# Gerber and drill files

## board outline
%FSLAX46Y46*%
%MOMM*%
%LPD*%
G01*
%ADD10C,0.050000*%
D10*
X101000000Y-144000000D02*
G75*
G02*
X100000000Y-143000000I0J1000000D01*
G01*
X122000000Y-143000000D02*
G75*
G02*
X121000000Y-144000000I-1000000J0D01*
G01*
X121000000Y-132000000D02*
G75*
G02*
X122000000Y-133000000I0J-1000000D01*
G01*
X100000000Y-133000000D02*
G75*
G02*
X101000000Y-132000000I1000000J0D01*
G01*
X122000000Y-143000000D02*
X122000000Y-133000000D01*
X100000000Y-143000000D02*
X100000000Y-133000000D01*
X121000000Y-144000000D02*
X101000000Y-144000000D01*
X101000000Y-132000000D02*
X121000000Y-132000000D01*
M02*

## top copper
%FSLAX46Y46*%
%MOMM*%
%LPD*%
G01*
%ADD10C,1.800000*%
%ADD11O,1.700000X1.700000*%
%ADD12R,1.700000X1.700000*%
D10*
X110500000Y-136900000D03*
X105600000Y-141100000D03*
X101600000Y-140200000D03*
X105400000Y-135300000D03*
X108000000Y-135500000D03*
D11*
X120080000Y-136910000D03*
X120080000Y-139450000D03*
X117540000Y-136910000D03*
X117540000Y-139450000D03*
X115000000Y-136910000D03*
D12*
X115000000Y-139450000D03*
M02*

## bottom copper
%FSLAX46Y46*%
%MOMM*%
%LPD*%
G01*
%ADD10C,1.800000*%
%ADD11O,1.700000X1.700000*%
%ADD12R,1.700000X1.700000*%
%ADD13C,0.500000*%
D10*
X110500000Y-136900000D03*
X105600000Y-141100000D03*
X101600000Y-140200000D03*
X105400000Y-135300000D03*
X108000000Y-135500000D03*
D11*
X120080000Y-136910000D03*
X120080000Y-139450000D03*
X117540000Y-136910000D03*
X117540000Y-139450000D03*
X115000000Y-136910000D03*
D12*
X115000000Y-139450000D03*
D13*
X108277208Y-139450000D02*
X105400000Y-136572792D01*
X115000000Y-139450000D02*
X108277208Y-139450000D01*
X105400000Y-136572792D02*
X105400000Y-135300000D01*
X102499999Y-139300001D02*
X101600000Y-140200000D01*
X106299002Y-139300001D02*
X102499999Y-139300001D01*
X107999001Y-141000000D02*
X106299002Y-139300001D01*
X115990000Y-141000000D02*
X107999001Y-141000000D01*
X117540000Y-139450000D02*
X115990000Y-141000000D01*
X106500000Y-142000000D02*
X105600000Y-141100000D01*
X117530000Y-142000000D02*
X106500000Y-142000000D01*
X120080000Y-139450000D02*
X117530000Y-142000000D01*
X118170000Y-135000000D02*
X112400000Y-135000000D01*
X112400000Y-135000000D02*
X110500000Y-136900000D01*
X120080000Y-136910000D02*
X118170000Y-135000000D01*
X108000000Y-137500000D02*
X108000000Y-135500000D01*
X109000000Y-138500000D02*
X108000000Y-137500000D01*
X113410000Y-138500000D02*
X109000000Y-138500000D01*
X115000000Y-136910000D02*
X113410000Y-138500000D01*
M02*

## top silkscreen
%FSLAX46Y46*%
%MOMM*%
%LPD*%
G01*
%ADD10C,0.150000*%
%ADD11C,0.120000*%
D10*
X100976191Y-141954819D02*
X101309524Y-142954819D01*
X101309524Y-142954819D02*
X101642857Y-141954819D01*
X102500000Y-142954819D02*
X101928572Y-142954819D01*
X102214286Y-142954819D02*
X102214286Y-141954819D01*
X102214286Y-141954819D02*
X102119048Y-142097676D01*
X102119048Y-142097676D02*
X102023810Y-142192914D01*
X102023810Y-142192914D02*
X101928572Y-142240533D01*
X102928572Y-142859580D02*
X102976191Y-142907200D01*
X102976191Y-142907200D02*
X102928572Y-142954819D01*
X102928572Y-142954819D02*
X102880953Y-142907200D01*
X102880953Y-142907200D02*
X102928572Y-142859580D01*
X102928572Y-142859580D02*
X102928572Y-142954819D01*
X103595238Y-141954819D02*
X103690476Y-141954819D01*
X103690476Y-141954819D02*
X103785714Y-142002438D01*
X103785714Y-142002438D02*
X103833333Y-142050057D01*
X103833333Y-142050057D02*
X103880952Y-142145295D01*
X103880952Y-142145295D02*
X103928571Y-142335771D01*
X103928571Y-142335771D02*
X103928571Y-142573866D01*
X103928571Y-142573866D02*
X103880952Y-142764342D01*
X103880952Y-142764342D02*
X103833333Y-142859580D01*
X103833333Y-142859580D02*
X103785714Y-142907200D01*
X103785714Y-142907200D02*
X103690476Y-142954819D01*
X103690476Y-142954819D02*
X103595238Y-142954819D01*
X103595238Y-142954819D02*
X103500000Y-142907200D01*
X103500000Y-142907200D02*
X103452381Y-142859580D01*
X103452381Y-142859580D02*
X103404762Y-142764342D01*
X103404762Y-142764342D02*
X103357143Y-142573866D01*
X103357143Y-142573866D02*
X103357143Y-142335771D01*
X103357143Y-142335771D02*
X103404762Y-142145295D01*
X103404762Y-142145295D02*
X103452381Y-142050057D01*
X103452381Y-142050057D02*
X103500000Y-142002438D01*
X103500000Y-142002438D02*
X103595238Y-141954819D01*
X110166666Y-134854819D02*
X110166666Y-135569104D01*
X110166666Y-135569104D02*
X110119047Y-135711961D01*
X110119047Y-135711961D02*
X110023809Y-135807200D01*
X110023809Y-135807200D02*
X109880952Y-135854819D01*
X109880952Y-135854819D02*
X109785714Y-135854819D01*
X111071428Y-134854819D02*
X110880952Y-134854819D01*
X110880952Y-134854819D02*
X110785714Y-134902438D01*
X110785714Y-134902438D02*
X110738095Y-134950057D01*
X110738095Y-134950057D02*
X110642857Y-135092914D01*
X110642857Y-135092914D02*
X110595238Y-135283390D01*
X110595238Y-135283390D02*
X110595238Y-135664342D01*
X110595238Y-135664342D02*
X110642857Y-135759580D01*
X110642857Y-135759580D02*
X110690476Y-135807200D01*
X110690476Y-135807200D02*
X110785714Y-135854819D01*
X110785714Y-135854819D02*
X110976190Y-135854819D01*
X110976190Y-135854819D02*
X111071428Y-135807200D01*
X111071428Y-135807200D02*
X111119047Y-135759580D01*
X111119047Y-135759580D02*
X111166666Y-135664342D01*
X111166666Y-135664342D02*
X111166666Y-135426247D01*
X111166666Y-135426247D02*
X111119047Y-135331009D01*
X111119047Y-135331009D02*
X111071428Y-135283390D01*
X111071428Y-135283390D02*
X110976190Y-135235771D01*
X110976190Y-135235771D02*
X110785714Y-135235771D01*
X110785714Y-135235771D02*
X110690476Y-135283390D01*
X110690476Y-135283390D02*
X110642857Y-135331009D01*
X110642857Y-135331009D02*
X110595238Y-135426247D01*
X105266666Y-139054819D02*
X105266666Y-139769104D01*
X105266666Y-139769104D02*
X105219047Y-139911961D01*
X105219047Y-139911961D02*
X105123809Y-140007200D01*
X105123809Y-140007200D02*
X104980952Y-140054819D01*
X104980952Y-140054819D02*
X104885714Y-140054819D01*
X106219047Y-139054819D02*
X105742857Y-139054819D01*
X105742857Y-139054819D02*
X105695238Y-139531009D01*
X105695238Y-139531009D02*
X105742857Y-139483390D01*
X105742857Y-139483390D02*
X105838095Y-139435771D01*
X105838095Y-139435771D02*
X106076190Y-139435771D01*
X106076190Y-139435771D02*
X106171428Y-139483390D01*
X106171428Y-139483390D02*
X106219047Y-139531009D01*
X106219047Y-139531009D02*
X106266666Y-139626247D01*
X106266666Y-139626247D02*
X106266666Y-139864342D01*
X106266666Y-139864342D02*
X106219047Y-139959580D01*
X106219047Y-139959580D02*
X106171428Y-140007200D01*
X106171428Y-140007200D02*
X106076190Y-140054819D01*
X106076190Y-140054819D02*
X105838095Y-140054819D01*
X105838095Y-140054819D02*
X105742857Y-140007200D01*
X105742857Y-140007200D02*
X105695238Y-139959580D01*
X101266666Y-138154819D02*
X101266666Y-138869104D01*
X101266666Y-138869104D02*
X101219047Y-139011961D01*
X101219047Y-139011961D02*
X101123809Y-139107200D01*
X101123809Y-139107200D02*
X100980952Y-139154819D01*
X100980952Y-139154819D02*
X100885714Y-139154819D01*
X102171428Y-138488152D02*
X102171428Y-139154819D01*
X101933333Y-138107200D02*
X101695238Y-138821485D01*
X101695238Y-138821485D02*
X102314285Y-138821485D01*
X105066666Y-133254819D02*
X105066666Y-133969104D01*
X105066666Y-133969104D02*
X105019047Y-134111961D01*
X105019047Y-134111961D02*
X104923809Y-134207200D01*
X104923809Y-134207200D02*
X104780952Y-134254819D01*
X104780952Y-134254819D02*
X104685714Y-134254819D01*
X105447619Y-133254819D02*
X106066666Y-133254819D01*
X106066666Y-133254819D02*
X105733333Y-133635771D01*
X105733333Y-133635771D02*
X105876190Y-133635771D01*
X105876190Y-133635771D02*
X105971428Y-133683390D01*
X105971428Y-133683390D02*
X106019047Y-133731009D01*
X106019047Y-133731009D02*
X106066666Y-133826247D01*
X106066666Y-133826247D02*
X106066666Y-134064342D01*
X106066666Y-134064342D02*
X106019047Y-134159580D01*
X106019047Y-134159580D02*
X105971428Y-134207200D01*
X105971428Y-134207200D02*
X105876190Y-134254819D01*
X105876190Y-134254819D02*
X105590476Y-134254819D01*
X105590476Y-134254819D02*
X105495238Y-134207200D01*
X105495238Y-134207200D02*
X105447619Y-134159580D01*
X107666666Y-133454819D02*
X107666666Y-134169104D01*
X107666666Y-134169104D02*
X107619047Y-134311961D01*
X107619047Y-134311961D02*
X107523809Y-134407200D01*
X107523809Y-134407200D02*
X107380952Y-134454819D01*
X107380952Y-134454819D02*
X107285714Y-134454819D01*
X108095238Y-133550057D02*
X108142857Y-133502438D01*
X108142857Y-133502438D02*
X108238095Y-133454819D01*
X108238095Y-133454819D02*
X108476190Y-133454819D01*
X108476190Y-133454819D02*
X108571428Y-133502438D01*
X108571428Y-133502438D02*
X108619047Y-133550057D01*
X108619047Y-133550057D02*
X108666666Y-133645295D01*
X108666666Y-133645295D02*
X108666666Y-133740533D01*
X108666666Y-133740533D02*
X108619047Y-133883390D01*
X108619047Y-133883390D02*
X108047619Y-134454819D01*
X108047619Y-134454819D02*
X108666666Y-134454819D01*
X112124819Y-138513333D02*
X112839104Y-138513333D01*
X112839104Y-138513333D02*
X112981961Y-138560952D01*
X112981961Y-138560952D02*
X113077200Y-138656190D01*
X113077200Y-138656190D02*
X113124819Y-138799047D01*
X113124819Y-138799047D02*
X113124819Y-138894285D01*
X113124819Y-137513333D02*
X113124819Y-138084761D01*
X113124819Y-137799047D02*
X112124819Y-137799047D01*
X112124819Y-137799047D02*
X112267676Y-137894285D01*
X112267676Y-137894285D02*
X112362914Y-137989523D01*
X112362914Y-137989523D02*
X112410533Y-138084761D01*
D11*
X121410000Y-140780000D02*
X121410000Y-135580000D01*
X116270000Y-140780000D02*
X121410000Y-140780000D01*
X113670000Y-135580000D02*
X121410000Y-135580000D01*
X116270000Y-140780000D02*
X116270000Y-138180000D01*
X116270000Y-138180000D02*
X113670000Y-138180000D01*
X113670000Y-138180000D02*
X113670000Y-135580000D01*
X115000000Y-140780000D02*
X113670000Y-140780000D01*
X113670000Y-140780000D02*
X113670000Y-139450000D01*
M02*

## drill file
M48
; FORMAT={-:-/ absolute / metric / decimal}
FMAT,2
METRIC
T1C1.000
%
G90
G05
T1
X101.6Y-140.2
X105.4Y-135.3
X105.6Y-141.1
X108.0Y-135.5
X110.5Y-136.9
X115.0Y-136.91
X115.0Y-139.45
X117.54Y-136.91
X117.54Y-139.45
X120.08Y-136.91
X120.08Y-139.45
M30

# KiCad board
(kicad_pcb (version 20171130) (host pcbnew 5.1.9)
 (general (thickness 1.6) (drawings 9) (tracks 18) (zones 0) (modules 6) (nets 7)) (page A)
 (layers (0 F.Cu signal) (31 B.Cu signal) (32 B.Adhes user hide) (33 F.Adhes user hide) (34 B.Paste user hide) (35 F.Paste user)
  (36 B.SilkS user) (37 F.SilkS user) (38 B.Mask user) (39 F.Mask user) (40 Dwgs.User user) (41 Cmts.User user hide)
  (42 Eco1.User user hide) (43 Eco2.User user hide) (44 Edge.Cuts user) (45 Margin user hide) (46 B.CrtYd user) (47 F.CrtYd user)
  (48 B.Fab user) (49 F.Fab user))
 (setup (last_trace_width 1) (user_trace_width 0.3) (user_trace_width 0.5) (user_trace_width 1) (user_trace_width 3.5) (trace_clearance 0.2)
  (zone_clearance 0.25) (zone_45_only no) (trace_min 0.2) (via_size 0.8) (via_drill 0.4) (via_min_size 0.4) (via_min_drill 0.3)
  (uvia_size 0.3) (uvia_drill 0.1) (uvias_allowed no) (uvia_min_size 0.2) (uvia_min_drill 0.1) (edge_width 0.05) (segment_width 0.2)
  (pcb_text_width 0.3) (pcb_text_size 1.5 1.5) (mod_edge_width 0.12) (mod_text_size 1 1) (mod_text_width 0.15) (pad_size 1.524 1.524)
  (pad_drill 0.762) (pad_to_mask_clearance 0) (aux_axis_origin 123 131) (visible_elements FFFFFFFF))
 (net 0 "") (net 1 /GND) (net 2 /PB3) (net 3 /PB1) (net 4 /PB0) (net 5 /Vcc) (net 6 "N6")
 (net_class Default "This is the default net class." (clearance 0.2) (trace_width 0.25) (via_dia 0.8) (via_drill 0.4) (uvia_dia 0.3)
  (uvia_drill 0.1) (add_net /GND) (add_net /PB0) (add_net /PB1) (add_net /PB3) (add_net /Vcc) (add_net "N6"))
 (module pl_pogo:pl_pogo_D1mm (layer F.Cu) (at 110.5 136.9)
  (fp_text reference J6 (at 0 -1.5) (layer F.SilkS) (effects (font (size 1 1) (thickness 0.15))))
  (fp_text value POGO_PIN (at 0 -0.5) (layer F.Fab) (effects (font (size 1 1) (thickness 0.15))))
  (pad 1 thru_hole circle (at 0 0) (size 1.8 1.8) (drill 1) (layers *.Cu *.Mask) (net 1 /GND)))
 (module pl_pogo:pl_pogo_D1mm (layer F.Cu) (at 105.6 141.1)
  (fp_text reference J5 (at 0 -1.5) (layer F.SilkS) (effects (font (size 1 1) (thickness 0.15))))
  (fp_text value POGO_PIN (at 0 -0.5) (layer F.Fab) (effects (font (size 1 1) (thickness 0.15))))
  (pad 1 thru_hole circle (at 0 0) (size 1.8 1.8) (drill 1) (layers *.Cu *.Mask) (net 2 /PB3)))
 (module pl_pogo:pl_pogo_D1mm (layer F.Cu) (at 101.6 140.2)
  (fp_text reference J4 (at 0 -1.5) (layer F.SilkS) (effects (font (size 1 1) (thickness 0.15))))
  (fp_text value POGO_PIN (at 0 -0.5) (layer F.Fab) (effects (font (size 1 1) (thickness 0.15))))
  (pad 1 thru_hole circle (at 0 0) (size 1.8 1.8) (drill 1) (layers *.Cu *.Mask) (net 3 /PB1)))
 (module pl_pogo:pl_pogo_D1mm (layer F.Cu) (at 105.4 135.3)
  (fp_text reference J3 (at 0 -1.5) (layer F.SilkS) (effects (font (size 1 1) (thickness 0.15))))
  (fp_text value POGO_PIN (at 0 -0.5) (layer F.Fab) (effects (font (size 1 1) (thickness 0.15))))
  (pad 1 thru_hole circle (at 0 0) (size 1.8 1.8) (drill 1) (layers *.Cu *.Mask) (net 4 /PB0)))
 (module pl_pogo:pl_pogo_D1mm (layer F.Cu) (at 108 135.5)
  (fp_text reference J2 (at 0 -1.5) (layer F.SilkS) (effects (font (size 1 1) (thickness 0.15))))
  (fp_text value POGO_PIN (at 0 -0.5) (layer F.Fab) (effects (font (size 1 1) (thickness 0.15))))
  (pad 1 thru_hole circle (at 0 0) (size 1.8 1.8) (drill 1) (layers *.Cu *.Mask) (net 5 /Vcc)))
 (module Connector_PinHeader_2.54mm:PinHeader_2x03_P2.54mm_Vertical (layer F.Cu) (at 115 139.45 90)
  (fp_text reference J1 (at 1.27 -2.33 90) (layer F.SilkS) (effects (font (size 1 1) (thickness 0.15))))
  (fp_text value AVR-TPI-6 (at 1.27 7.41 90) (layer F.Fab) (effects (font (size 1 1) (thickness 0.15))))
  (fp_line (start -1.33 6.41) (end 3.87 6.41) (layer F.SilkS) (width 0.12))
  (fp_line (start -1.33 1.27) (end -1.33 6.41) (layer F.SilkS) (width 0.12))
  (fp_line (start 3.87 -1.33) (end 3.87 6.41) (layer F.SilkS) (width 0.12))
  (fp_line (start -1.33 1.27) (end 1.27 1.27) (layer F.SilkS) (width 0.12))
  (fp_line (start 1.27 1.27) (end 1.27 -1.33) (layer F.SilkS) (width 0.12))
  (fp_line (start 1.27 -1.33) (end 3.87 -1.33) (layer F.SilkS) (width 0.12))
  (fp_line (start -1.33 0) (end -1.33 -1.33) (layer F.SilkS) (width 0.12))
  (fp_line (start -1.33 -1.33) (end 0 -1.33) (layer F.SilkS) (width 0.12))
  (pad 6 thru_hole oval (at 2.54 5.08 90) (size 1.7 1.7) (drill 1) (layers *.Cu *.Mask) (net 1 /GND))
  (pad 5 thru_hole oval (at 0 5.08 90) (size 1.7 1.7) (drill 1) (layers *.Cu *.Mask) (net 2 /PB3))
  (pad 4 thru_hole oval (at 2.54 2.54 90) (size 1.7 1.7) (drill 1) (layers *.Cu *.Mask) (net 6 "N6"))
  (pad 3 thru_hole oval (at 0 2.54 90) (size 1.7 1.7) (drill 1) (layers *.Cu *.Mask) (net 3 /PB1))
  (pad 2 thru_hole oval (at 2.54 0 90) (size 1.7 1.7) (drill 1) (layers *.Cu *.Mask) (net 5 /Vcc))
  (pad 1 thru_hole rect (at 0 0 90) (size 1.7 1.7) (drill 1) (layers *.Cu *.Mask) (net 4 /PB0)))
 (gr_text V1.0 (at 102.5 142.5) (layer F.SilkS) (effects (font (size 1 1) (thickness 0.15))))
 (gr_arc (start 101 143) (end 100 143) (angle -90) (layer Edge.Cuts) (width 0.05))
 (gr_arc (start 121 143) (end 121 144) (angle -90) (layer Edge.Cuts) (width 0.05))
 (gr_arc (start 121 133) (end 122 133) (angle -90) (layer Edge.Cuts) (width 0.05))
 (gr_arc (start 101 133) (end 101 132) (angle -90) (layer Edge.Cuts) (width 0.05))
 (gr_line (start 122 143) (end 122 133) (layer Edge.Cuts) (width 0.05))
 (gr_line (start 100 143) (end 100 133) (layer Edge.Cuts) (width 0.05))
 (gr_line (start 121 144) (end 101 144) (layer Edge.Cuts) (width 0.05))
 (gr_line (start 101 132) (end 121 132) (layer Edge.Cuts) (width 0.05))
 (segment (start 108.277208 139.45) (end 105.4 136.572792) (width 0.5) (layer B.Cu) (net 4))
 (segment (start 115 139.45) (end 108.277208 139.45) (width 0.5) (layer B.Cu) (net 4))
 (segment (start 105.4 136.572792) (end 105.4 135.3) (width 0.5) (layer B.Cu) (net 4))
 (segment (start 102.499999 139.300001) (end 101.6 140.2) (width 0.5) (layer B.Cu) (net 3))
 (segment (start 106.299002 139.300001) (end 102.499999 139.300001) (width 0.5) (layer B.Cu) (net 3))
 (segment (start 107.999001 141) (end 106.299002 139.300001) (width 0.5) (layer B.Cu) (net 3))
 (segment (start 115.99 141) (end 107.999001 141) (width 0.5) (layer B.Cu) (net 3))
 (segment (start 117.54 139.45) (end 115.99 141) (width 0.5) (layer B.Cu) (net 3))
 (segment (start 106.5 142) (end 105.6 141.1) (width 0.5) (layer B.Cu) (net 2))
 (segment (start 117.53 142) (end 106.5 142) (width 0.5) (layer B.Cu) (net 2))
 (segment (start 120.08 139.45) (end 117.53 142) (width 0.5) (layer B.Cu) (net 2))
 (segment (start 118.17 135) (end 112.4 135) (width 0.5) (layer B.Cu) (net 1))
 (segment (start 112.4 135) (end 110.5 136.9) (width 0.5) (layer B.Cu) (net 1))
 (segment (start 120.08 136.91) (end 118.17 135) (width 0.5) (layer B.Cu) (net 1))
 (segment (start 108 137.5) (end 108 135.5) (width 0.5) (layer B.Cu) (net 5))
 (segment (start 109 138.5) (end 108 137.5) (width 0.5) (layer B.Cu) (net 5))
 (segment (start 113.41 138.5) (end 109 138.5) (width 0.5) (layer B.Cu) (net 5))
 (segment (start 115 136.91) (end 113.41 138.5) (width 0.5) (layer B.Cu) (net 5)))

